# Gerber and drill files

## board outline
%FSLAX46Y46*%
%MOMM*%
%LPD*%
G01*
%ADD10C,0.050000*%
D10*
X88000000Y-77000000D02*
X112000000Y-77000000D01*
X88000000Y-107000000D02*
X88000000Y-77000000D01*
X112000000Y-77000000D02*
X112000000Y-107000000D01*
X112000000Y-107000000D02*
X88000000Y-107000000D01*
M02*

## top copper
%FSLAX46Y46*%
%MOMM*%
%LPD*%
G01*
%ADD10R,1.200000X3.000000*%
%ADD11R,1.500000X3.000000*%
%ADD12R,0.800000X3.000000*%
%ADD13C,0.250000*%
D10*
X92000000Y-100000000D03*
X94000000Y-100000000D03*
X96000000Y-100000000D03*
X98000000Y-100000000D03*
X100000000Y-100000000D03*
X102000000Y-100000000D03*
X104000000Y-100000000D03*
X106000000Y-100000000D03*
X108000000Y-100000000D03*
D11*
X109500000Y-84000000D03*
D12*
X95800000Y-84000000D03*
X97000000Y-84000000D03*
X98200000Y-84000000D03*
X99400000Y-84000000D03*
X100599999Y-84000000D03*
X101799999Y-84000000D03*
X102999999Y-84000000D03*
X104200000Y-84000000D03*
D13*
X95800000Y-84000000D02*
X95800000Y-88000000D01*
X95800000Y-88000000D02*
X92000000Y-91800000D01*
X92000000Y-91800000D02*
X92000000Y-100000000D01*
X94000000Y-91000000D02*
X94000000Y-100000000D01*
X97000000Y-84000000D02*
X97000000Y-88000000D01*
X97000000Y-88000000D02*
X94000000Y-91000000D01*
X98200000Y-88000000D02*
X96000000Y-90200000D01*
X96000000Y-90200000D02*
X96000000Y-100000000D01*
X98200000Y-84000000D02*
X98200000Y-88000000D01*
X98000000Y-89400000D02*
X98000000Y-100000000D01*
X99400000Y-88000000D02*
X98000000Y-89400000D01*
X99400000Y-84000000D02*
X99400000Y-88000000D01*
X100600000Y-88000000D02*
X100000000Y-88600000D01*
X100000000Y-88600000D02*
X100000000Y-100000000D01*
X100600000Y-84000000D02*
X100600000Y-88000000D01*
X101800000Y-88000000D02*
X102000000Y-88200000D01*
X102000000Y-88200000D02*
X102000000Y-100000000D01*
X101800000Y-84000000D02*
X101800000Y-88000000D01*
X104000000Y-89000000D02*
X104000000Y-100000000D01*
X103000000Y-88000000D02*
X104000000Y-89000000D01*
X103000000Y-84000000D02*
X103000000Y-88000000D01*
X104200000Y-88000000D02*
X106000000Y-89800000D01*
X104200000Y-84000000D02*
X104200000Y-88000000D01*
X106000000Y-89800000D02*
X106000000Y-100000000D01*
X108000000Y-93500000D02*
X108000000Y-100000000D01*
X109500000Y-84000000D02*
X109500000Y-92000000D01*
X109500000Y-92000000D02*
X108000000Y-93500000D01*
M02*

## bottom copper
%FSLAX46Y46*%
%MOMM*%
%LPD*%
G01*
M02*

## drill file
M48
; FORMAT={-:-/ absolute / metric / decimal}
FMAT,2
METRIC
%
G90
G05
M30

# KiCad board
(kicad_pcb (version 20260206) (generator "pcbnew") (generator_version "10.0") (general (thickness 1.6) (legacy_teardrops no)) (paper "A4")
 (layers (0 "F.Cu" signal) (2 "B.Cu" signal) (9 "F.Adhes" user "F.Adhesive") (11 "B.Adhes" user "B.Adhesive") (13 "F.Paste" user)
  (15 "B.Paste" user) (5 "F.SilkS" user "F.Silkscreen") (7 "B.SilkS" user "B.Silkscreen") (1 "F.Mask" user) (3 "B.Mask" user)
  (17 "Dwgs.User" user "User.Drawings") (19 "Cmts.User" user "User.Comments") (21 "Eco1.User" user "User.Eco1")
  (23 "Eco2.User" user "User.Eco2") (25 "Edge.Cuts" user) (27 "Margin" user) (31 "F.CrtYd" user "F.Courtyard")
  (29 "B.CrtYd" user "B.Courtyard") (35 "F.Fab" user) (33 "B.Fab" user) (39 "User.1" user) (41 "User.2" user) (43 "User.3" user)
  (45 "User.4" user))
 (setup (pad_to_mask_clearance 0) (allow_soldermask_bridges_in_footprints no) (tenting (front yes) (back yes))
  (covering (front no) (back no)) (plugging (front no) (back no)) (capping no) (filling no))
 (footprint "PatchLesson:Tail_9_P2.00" (layer "F.Cu") (at 100 100)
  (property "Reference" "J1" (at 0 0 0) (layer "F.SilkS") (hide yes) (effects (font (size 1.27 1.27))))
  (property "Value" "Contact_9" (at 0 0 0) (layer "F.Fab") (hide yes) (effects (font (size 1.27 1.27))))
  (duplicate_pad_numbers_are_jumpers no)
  (pad "1" smd rect (at -8 0) (size 1.2 3) (layers "F.Cu" "F.Mask") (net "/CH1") (solder_mask_margin 0.05) (thermal_bridge_angle 45))
  (pad "2" smd rect (at -6 0) (size 1.2 3) (layers "F.Cu" "F.Mask") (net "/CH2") (solder_mask_margin 0.05) (thermal_bridge_angle 45))
  (pad "3" smd rect (at -4 0) (size 1.2 3) (layers "F.Cu" "F.Mask") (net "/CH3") (solder_mask_margin 0.05) (thermal_bridge_angle 45))
  (pad "4" smd rect (at -2 0) (size 1.2 3) (layers "F.Cu" "F.Mask") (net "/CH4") (solder_mask_margin 0.05) (thermal_bridge_angle 45))
  (pad "5" smd rect (at 0 0) (size 1.2 3) (layers "F.Cu" "F.Mask") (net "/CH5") (solder_mask_margin 0.05) (thermal_bridge_angle 45))
  (pad "6" smd rect (at 2 0) (size 1.2 3) (layers "F.Cu" "F.Mask") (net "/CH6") (solder_mask_margin 0.05) (thermal_bridge_angle 45))
  (pad "7" smd rect (at 4 0) (size 1.2 3) (layers "F.Cu" "F.Mask") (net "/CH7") (solder_mask_margin 0.05) (thermal_bridge_angle 45))
  (pad "8" smd rect (at 6 0) (size 1.2 3) (layers "F.Cu" "F.Mask") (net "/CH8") (solder_mask_margin 0.05) (thermal_bridge_angle 45))
  (pad "9" smd rect (at 8 0) (size 1.2 3) (layers "F.Cu" "F.Mask") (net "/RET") (solder_mask_margin 0.05) (thermal_bridge_angle 45)))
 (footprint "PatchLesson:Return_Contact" (layer "F.Cu") (at 109.5 84)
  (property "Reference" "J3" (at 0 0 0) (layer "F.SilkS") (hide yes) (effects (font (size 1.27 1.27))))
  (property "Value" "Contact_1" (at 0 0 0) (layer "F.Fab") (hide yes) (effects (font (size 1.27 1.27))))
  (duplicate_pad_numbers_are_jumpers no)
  (pad "1" smd rect (at 0 0) (size 1.5 3) (layers "F.Cu" "F.Mask") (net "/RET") (solder_mask_margin 0.05) (thermal_bridge_angle 45)))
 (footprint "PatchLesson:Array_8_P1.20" (layer "F.Cu") (at 100 84)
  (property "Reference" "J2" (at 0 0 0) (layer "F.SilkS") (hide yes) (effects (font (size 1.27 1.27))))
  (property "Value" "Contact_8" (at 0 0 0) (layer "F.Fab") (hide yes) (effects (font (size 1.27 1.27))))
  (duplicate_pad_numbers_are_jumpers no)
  (pad "1" smd rect (at -4.2 0) (size 0.8 3) (layers "F.Cu" "F.Mask") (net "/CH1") (solder_mask_margin 0.05) (thermal_bridge_angle 45))
  (pad "2" smd rect (at -3 0) (size 0.8 3) (layers "F.Cu" "F.Mask") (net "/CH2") (solder_mask_margin 0.05) (thermal_bridge_angle 45))
  (pad "3" smd rect (at -1.8 0) (size 0.8 3) (layers "F.Cu" "F.Mask") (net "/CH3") (solder_mask_margin 0.05) (thermal_bridge_angle 45))
  (pad "4" smd rect (at -0.6 0) (size 0.8 3) (layers "F.Cu" "F.Mask") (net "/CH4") (solder_mask_margin 0.05) (thermal_bridge_angle 45))
  (pad "5" smd rect (at 0.599999 0) (size 0.8 3) (layers "F.Cu" "F.Mask") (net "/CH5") (solder_mask_margin 0.05) (thermal_bridge_angle 45))
  (pad "6" smd rect (at 1.799999 0) (size 0.8 3) (layers "F.Cu" "F.Mask") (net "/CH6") (solder_mask_margin 0.05) (thermal_bridge_angle 45))
  (pad "7" smd rect (at 2.999999 0) (size 0.8 3) (layers "F.Cu" "F.Mask") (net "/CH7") (solder_mask_margin 0.05) (thermal_bridge_angle 45))
  (pad "8" smd rect (at 4.2 0) (size 0.8 3) (layers "F.Cu" "F.Mask") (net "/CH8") (solder_mask_margin 0.05) (thermal_bridge_angle 45)))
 (gr_line (start 88 77) (end 112 77) (stroke (width 0.05) (type default)) (layer "Edge.Cuts"))
 (gr_line (start 88 107) (end 88 77) (stroke (width 0.05) (type default)) (layer "Edge.Cuts"))
 (gr_line (start 112 77) (end 112 107) (stroke (width 0.05) (type default)) (layer "Edge.Cuts"))
 (gr_line (start 112 107) (end 88 107) (stroke (width 0.05) (type default)) (layer "Edge.Cuts"))
 (segment (start 95.8 84) (end 95.8 88) (width 0.25) (layer "F.Cu") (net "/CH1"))
 (segment (start 95.8 88) (end 92 91.8) (width 0.25) (layer "F.Cu") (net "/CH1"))
 (segment (start 92 91.8) (end 92 100) (width 0.25) (layer "F.Cu") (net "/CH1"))
 (segment (start 94 91) (end 94 100) (width 0.25) (layer "F.Cu") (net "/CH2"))
 (segment (start 97 84) (end 97 88) (width 0.25) (layer "F.Cu") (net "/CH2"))
 (segment (start 97 88) (end 94 91) (width 0.25) (layer "F.Cu") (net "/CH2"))
 (segment (start 98.2 88) (end 96 90.2) (width 0.25) (layer "F.Cu") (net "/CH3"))
 (segment (start 96 90.2) (end 96 100) (width 0.25) (layer "F.Cu") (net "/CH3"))
 (segment (start 98.2 84) (end 98.2 88) (width 0.25) (layer "F.Cu") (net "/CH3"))
 (segment (start 98 89.4) (end 98 100) (width 0.25) (layer "F.Cu") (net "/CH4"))
 (segment (start 99.4 88) (end 98 89.4) (width 0.25) (layer "F.Cu") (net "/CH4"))
 (segment (start 99.4 84) (end 99.4 88) (width 0.25) (layer "F.Cu") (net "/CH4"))
 (segment (start 100.6 88) (end 100 88.6) (width 0.25) (layer "F.Cu") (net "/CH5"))
 (segment (start 100 88.6) (end 100 100) (width 0.25) (layer "F.Cu") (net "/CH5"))
 (segment (start 100.6 84) (end 100.6 88) (width 0.25) (layer "F.Cu") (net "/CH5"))
 (segment (start 101.8 88) (end 102 88.2) (width 0.25) (layer "F.Cu") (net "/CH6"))
 (segment (start 102 88.2) (end 102 100) (width 0.25) (layer "F.Cu") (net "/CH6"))
 (segment (start 101.8 84) (end 101.8 88) (width 0.25) (layer "F.Cu") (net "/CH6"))
 (segment (start 104 89) (end 104 100) (width 0.25) (layer "F.Cu") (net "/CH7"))
 (segment (start 103 88) (end 104 89) (width 0.25) (layer "F.Cu") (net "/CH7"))
 (segment (start 103 84) (end 103 88) (width 0.25) (layer "F.Cu") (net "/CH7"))
 (segment (start 104.2 88) (end 106 89.8) (width 0.25) (layer "F.Cu") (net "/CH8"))
 (segment (start 104.2 84) (end 104.2 88) (width 0.25) (layer "F.Cu") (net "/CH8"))
 (segment (start 106 89.8) (end 106 100) (width 0.25) (layer "F.Cu") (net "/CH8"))
 (segment (start 108 93.5) (end 108 100) (width 0.25) (layer "F.Cu") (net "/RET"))
 (segment (start 109.5 84) (end 109.5 92) (width 0.25) (layer "F.Cu") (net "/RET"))
 (segment (start 109.5 92) (end 108 93.5) (width 0.25) (layer "F.Cu") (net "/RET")))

